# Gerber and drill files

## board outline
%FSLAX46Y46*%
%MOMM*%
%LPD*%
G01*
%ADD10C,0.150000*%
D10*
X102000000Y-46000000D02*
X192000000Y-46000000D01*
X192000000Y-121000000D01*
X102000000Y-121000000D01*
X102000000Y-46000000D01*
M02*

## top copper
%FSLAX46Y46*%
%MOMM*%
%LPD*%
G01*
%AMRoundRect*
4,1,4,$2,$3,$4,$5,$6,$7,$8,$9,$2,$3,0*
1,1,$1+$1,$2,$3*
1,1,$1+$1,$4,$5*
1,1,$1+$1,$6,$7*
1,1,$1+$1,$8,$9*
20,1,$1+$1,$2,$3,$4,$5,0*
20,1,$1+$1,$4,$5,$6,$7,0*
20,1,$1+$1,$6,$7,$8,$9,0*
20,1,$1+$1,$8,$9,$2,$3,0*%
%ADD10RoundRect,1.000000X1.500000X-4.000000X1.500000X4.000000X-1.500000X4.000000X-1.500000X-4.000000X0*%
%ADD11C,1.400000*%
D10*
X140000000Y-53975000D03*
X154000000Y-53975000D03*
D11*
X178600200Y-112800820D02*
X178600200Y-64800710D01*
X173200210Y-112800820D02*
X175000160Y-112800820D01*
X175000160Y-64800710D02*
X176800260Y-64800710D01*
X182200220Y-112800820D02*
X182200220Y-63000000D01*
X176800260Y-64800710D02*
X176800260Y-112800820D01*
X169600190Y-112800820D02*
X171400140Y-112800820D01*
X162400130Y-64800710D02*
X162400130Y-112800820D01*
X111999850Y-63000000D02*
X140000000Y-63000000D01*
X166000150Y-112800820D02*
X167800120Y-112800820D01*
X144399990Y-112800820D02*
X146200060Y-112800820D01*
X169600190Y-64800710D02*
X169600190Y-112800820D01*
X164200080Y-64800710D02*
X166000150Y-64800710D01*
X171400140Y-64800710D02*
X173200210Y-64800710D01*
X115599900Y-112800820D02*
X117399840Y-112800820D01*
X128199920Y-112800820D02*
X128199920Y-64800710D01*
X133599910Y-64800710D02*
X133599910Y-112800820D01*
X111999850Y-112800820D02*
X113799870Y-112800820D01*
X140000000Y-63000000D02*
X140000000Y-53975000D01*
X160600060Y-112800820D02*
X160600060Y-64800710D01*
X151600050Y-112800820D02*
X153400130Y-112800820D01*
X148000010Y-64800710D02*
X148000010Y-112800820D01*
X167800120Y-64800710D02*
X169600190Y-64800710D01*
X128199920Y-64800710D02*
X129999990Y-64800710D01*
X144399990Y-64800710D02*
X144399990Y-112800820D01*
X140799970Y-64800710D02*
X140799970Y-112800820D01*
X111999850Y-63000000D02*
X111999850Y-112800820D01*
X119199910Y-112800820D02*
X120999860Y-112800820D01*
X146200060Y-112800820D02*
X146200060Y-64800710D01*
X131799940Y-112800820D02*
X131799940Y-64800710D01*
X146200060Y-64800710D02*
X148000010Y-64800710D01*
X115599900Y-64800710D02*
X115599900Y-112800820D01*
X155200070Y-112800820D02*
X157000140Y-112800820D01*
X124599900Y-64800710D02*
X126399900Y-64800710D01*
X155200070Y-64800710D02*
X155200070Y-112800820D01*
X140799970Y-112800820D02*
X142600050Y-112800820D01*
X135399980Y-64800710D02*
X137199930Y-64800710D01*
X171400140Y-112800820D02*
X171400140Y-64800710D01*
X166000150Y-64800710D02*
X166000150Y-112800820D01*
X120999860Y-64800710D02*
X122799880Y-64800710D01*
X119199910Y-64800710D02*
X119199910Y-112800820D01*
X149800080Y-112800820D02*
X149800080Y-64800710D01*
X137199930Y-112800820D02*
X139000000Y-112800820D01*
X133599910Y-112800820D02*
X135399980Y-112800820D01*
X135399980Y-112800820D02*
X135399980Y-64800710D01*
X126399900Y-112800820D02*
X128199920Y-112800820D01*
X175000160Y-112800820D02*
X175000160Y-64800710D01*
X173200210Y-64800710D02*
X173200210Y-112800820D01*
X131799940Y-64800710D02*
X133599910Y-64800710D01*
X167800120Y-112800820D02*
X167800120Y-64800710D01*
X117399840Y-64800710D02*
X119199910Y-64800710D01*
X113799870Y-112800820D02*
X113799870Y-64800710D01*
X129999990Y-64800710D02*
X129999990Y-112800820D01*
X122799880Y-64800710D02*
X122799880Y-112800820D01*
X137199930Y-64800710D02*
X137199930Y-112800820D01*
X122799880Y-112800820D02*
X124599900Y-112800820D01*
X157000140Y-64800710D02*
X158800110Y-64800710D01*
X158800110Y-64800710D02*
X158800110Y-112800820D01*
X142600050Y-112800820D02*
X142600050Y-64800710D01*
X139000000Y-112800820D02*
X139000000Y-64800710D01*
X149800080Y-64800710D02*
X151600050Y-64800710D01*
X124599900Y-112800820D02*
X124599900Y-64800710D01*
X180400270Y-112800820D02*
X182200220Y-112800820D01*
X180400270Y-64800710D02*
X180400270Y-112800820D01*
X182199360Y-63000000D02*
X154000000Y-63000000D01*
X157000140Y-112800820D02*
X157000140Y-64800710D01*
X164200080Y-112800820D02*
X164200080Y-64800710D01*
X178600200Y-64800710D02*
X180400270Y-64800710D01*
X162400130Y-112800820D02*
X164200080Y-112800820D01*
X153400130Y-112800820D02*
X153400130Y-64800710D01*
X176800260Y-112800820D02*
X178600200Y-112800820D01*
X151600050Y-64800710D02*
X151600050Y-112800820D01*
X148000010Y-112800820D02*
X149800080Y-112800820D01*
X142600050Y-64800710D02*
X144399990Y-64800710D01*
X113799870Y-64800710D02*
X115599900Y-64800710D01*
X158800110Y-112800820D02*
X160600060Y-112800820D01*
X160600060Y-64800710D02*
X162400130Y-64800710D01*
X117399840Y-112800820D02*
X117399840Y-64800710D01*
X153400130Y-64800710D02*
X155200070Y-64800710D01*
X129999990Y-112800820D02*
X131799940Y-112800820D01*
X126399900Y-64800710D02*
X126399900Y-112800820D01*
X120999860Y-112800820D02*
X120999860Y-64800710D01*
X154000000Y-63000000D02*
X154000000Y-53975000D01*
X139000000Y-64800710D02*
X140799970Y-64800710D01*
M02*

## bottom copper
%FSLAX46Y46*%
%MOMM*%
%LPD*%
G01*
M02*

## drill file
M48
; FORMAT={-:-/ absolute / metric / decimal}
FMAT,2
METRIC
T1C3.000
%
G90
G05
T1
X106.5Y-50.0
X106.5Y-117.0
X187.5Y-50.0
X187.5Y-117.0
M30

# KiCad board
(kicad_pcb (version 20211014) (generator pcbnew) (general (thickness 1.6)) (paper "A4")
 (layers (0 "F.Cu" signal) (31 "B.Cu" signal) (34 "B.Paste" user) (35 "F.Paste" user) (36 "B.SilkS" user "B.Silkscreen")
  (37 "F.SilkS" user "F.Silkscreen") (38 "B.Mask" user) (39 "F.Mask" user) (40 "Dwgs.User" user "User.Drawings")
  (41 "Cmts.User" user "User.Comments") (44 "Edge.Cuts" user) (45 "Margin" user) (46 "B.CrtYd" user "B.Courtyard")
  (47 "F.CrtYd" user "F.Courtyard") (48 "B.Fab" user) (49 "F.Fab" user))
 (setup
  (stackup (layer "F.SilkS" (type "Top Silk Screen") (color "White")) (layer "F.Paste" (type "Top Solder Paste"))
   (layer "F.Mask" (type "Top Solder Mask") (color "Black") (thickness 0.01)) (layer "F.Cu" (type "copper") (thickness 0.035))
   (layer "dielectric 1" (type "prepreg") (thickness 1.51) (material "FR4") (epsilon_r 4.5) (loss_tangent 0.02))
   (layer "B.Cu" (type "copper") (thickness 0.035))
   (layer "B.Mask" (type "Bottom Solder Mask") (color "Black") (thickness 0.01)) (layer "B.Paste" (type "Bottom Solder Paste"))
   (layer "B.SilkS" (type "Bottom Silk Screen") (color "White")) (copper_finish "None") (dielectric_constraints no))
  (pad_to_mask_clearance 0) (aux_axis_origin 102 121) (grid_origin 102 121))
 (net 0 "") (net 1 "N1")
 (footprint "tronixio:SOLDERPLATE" (layer "F.Cu") (at 147 113.975)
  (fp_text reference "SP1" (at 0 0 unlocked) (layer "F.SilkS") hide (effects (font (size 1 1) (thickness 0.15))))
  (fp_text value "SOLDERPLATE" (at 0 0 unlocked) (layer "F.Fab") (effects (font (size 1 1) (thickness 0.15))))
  (pad "1" smd roundrect (at -7 -60 90) (size 10 5) (layers "F.Cu" "F.Paste" "F.Mask") (roundrect_rratio 0.2) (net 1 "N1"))
  (pad "1" smd roundrect (at 7 -60 90) (size 10 5) (layers "F.Cu" "F.Paste" "F.Mask") (roundrect_rratio 0.2) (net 1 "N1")))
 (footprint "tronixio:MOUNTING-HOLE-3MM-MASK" (layer "F.Cu") (at 106.5 50)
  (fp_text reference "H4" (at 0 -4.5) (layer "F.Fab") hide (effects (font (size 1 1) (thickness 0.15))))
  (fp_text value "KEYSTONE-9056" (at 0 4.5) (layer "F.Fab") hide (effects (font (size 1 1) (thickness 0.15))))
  (pad "" np_thru_hole circle (at 0 0) (size 3 3) (drill 3) (layers F&B.Cu *.Mask) (solder_mask_margin 1.5) (clearance 1.5)))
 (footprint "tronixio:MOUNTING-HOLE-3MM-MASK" (layer "F.Cu") (at 106.5 117)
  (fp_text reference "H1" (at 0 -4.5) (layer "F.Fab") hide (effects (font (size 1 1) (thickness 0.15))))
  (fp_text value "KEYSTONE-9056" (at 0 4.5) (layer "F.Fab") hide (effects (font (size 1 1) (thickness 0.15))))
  (pad "" np_thru_hole circle (at 0 0) (size 3 3) (drill 3) (layers F&B.Cu *.Mask) (solder_mask_margin 1.5) (clearance 1.5)))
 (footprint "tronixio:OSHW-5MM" (layer "F.Cu") (at 113.5 50)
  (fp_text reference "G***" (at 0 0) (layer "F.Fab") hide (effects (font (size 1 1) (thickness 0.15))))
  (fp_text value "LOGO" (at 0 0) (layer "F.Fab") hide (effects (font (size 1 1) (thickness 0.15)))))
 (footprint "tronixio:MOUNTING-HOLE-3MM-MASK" (layer "F.Cu") (at 187.5 117)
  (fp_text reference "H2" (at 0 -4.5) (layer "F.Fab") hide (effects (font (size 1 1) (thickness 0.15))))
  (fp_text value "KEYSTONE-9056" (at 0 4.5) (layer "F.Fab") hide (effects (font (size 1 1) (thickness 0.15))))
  (pad "" np_thru_hole circle (at 0 0) (size 3 3) (drill 3) (layers F&B.Cu *.Mask) (solder_mask_margin 1.5) (clearance 1.5)))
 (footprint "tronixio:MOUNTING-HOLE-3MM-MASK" (layer "F.Cu") (at 187.5 50)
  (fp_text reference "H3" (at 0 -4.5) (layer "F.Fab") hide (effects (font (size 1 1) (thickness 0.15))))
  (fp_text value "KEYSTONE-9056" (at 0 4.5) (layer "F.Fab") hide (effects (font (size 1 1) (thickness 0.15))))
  (pad "" np_thru_hole circle (at 0 0) (size 3 3) (drill 3) (layers F&B.Cu *.Mask) (solder_mask_margin 1.5) (clearance 1.5)))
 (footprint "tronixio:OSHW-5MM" (layer "B.Cu") (at 113.5 50 180)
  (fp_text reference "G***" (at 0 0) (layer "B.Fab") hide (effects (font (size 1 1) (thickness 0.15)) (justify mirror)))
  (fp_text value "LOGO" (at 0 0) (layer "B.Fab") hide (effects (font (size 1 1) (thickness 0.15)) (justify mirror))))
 (gr_rect (start 102 121) (end 192 46) (layer "Edge.Cuts") (width 0.15) (fill none))
 (segment (start 178.6002 112.80082) (end 178.6002 64.80071) (width 1.4) (layer "F.Cu") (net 1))
 (segment (start 173.20021 112.80082) (end 175.00016 112.80082) (width 1.4) (layer "F.Cu") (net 1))
 (segment (start 175.00016 64.80071) (end 176.80026 64.80071) (width 1.4) (layer "F.Cu") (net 1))
 (segment (start 182.20022 112.80082) (end 182.20022 63) (width 1.4) (layer "F.Cu") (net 1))
 (segment (start 176.80026 64.80071) (end 176.80026 112.80082) (width 1.4) (layer "F.Cu") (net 1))
 (segment (start 169.60019 112.80082) (end 171.40014 112.80082) (width 1.4) (layer "F.Cu") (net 1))
 (segment (start 162.40013 64.80071) (end 162.40013 112.80082) (width 1.4) (layer "F.Cu") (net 1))
 (segment (start 111.99985 63) (end 140 63) (width 1.4) (layer "F.Cu") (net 1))
 (segment (start 166.00015 112.80082) (end 167.80012 112.80082) (width 1.4) (layer "F.Cu") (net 1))
 (segment (start 144.39999 112.80082) (end 146.20006 112.80082) (width 1.4) (layer "F.Cu") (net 1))
 (segment (start 169.60019 64.80071) (end 169.60019 112.80082) (width 1.4) (layer "F.Cu") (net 1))
 (segment (start 164.20008 64.80071) (end 166.00015 64.80071) (width 1.4) (layer "F.Cu") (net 1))
 (segment (start 171.40014 64.80071) (end 173.20021 64.80071) (width 1.4) (layer "F.Cu") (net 1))
 (segment (start 115.5999 112.80082) (end 117.39984 112.80082) (width 1.4) (layer "F.Cu") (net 1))
 (segment (start 128.19992 112.80082) (end 128.19992 64.80071) (width 1.4) (layer "F.Cu") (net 1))
 (segment (start 133.59991 64.80071) (end 133.59991 112.80082) (width 1.4) (layer "F.Cu") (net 1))
 (segment (start 111.99985 112.80082) (end 113.79987 112.80082) (width 1.4) (layer "F.Cu") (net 1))
 (segment (start 140 63) (end 140 53.975) (width 1.4) (layer "F.Cu") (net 1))
 (segment (start 160.60006 112.80082) (end 160.60006 64.80071) (width 1.4) (layer "F.Cu") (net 1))
 (segment (start 151.60005 112.80082) (end 153.40013 112.80082) (width 1.4) (layer "F.Cu") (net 1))
 (segment (start 148.00001 64.80071) (end 148.00001 112.80082) (width 1.4) (layer "F.Cu") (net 1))
 (segment (start 167.80012 64.80071) (end 169.60019 64.80071) (width 1.4) (layer "F.Cu") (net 1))
 (segment (start 128.19992 64.80071) (end 129.99999 64.80071) (width 1.4) (layer "F.Cu") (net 1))
 (segment (start 144.39999 64.80071) (end 144.39999 112.80082) (width 1.4) (layer "F.Cu") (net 1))
 (segment (start 140.79997 64.80071) (end 140.79997 112.80082) (width 1.4) (layer "F.Cu") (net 1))
 (segment (start 111.99985 63) (end 111.99985 112.80082) (width 1.4) (layer "F.Cu") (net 1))
 (segment (start 119.19991 112.80082) (end 120.99986 112.80082) (width 1.4) (layer "F.Cu") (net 1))
 (segment (start 146.20006 112.80082) (end 146.20006 64.80071) (width 1.4) (layer "F.Cu") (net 1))
 (segment (start 131.79994 112.80082) (end 131.79994 64.80071) (width 1.4) (layer "F.Cu") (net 1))
 (segment (start 146.20006 64.80071) (end 148.00001 64.80071) (width 1.4) (layer "F.Cu") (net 1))
 (segment (start 115.5999 64.80071) (end 115.5999 112.80082) (width 1.4) (layer "F.Cu") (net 1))
 (segment (start 155.20007 112.80082) (end 157.00014 112.80082) (width 1.4) (layer "F.Cu") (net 1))
 (segment (start 124.5999 64.80071) (end 126.3999 64.80071) (width 1.4) (layer "F.Cu") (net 1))
 (segment (start 155.20007 64.80071) (end 155.20007 112.80082) (width 1.4) (layer "F.Cu") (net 1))
 (segment (start 140.79997 112.80082) (end 142.60005 112.80082) (width 1.4) (layer "F.Cu") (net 1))
 (segment (start 135.39998 64.80071) (end 137.19993 64.80071) (width 1.4) (layer "F.Cu") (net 1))
 (segment (start 171.40014 112.80082) (end 171.40014 64.80071) (width 1.4) (layer "F.Cu") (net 1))
 (segment (start 166.00015 64.80071) (end 166.00015 112.80082) (width 1.4) (layer "F.Cu") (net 1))
 (segment (start 120.99986 64.80071) (end 122.79988 64.80071) (width 1.4) (layer "F.Cu") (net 1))
 (segment (start 119.19991 64.80071) (end 119.19991 112.80082) (width 1.4) (layer "F.Cu") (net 1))
 (segment (start 149.80008 112.80082) (end 149.80008 64.80071) (width 1.4) (layer "F.Cu") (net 1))
 (segment (start 137.19993 112.80082) (end 139 112.80082) (width 1.4) (layer "F.Cu") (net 1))
 (segment (start 133.59991 112.80082) (end 135.39998 112.80082) (width 1.4) (layer "F.Cu") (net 1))
 (segment (start 135.39998 112.80082) (end 135.39998 64.80071) (width 1.4) (layer "F.Cu") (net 1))
 (segment (start 126.3999 112.80082) (end 128.19992 112.80082) (width 1.4) (layer "F.Cu") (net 1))
 (segment (start 175.00016 112.80082) (end 175.00016 64.80071) (width 1.4) (layer "F.Cu") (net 1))
 (segment (start 173.20021 64.80071) (end 173.20021 112.80082) (width 1.4) (layer "F.Cu") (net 1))
 (segment (start 131.79994 64.80071) (end 133.59991 64.80071) (width 1.4) (layer "F.Cu") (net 1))
 (segment (start 167.80012 112.80082) (end 167.80012 64.80071) (width 1.4) (layer "F.Cu") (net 1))
 (segment (start 117.39984 64.80071) (end 119.19991 64.80071) (width 1.4) (layer "F.Cu") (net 1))
 (segment (start 113.79987 112.80082) (end 113.79987 64.80071) (width 1.4) (layer "F.Cu") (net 1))
 (segment (start 129.99999 64.80071) (end 129.99999 112.80082) (width 1.4) (layer "F.Cu") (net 1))
 (segment (start 122.79988 64.80071) (end 122.79988 112.80082) (width 1.4) (layer "F.Cu") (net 1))
 (segment (start 137.19993 64.80071) (end 137.19993 112.80082) (width 1.4) (layer "F.Cu") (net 1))
 (segment (start 122.79988 112.80082) (end 124.5999 112.80082) (width 1.4) (layer "F.Cu") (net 1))
 (segment (start 157.00014 64.80071) (end 158.80011 64.80071) (width 1.4) (layer "F.Cu") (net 1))
 (segment (start 158.80011 64.80071) (end 158.80011 112.80082) (width 1.4) (layer "F.Cu") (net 1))
 (segment (start 142.60005 112.80082) (end 142.60005 64.80071) (width 1.4) (layer "F.Cu") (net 1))
 (segment (start 139 112.80082) (end 139 64.80071) (width 1.4) (layer "F.Cu") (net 1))
 (segment (start 149.80008 64.80071) (end 151.60005 64.80071) (width 1.4) (layer "F.Cu") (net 1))
 (segment (start 124.5999 112.80082) (end 124.5999 64.80071) (width 1.4) (layer "F.Cu") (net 1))
 (segment (start 180.40027 112.80082) (end 182.20022 112.80082) (width 1.4) (layer "F.Cu") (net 1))
 (segment (start 180.40027 64.80071) (end 180.40027 112.80082) (width 1.4) (layer "F.Cu") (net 1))
 (segment (start 182.19936 63) (end 154 63) (width 1.4) (layer "F.Cu") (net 1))
 (segment (start 157.00014 112.80082) (end 157.00014 64.80071) (width 1.4) (layer "F.Cu") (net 1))
 (segment (start 164.20008 112.80082) (end 164.20008 64.80071) (width 1.4) (layer "F.Cu") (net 1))
 (segment (start 178.6002 64.80071) (end 180.40027 64.80071) (width 1.4) (layer "F.Cu") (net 1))
 (segment (start 162.40013 112.80082) (end 164.20008 112.80082) (width 1.4) (layer "F.Cu") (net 1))
 (segment (start 153.40013 112.80082) (end 153.40013 64.80071) (width 1.4) (layer "F.Cu") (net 1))
 (segment (start 176.80026 112.80082) (end 178.6002 112.80082) (width 1.4) (layer "F.Cu") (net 1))
 (segment (start 151.60005 64.80071) (end 151.60005 112.80082) (width 1.4) (layer "F.Cu") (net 1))
 (segment (start 148.00001 112.80082) (end 149.80008 112.80082) (width 1.4) (layer "F.Cu") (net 1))
 (segment (start 142.60005 64.80071) (end 144.39999 64.80071) (width 1.4) (layer "F.Cu") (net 1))
 (segment (start 113.79987 64.80071) (end 115.5999 64.80071) (width 1.4) (layer "F.Cu") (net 1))
 (segment (start 158.80011 112.80082) (end 160.60006 112.80082) (width 1.4) (layer "F.Cu") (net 1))
 (segment (start 160.60006 64.80071) (end 162.40013 64.80071) (width 1.4) (layer "F.Cu") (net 1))
 (segment (start 117.39984 112.80082) (end 117.39984 64.80071) (width 1.4) (layer "F.Cu") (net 1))
 (segment (start 153.40013 64.80071) (end 155.20007 64.80071) (width 1.4) (layer "F.Cu") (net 1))
 (segment (start 129.99999 112.80082) (end 131.79994 112.80082) (width 1.4) (layer "F.Cu") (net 1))
 (segment (start 126.3999 64.80071) (end 126.3999 112.80082) (width 1.4) (layer "F.Cu") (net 1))
 (segment (start 120.99986 112.80082) (end 120.99986 64.80071) (width 1.4) (layer "F.Cu") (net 1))
 (segment (start 154 63) (end 154 53.975) (width 1.4) (layer "F.Cu") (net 1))
 (segment (start 139 64.80071) (end 140.79997 64.80071) (width 1.4) (layer "F.Cu") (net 1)))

